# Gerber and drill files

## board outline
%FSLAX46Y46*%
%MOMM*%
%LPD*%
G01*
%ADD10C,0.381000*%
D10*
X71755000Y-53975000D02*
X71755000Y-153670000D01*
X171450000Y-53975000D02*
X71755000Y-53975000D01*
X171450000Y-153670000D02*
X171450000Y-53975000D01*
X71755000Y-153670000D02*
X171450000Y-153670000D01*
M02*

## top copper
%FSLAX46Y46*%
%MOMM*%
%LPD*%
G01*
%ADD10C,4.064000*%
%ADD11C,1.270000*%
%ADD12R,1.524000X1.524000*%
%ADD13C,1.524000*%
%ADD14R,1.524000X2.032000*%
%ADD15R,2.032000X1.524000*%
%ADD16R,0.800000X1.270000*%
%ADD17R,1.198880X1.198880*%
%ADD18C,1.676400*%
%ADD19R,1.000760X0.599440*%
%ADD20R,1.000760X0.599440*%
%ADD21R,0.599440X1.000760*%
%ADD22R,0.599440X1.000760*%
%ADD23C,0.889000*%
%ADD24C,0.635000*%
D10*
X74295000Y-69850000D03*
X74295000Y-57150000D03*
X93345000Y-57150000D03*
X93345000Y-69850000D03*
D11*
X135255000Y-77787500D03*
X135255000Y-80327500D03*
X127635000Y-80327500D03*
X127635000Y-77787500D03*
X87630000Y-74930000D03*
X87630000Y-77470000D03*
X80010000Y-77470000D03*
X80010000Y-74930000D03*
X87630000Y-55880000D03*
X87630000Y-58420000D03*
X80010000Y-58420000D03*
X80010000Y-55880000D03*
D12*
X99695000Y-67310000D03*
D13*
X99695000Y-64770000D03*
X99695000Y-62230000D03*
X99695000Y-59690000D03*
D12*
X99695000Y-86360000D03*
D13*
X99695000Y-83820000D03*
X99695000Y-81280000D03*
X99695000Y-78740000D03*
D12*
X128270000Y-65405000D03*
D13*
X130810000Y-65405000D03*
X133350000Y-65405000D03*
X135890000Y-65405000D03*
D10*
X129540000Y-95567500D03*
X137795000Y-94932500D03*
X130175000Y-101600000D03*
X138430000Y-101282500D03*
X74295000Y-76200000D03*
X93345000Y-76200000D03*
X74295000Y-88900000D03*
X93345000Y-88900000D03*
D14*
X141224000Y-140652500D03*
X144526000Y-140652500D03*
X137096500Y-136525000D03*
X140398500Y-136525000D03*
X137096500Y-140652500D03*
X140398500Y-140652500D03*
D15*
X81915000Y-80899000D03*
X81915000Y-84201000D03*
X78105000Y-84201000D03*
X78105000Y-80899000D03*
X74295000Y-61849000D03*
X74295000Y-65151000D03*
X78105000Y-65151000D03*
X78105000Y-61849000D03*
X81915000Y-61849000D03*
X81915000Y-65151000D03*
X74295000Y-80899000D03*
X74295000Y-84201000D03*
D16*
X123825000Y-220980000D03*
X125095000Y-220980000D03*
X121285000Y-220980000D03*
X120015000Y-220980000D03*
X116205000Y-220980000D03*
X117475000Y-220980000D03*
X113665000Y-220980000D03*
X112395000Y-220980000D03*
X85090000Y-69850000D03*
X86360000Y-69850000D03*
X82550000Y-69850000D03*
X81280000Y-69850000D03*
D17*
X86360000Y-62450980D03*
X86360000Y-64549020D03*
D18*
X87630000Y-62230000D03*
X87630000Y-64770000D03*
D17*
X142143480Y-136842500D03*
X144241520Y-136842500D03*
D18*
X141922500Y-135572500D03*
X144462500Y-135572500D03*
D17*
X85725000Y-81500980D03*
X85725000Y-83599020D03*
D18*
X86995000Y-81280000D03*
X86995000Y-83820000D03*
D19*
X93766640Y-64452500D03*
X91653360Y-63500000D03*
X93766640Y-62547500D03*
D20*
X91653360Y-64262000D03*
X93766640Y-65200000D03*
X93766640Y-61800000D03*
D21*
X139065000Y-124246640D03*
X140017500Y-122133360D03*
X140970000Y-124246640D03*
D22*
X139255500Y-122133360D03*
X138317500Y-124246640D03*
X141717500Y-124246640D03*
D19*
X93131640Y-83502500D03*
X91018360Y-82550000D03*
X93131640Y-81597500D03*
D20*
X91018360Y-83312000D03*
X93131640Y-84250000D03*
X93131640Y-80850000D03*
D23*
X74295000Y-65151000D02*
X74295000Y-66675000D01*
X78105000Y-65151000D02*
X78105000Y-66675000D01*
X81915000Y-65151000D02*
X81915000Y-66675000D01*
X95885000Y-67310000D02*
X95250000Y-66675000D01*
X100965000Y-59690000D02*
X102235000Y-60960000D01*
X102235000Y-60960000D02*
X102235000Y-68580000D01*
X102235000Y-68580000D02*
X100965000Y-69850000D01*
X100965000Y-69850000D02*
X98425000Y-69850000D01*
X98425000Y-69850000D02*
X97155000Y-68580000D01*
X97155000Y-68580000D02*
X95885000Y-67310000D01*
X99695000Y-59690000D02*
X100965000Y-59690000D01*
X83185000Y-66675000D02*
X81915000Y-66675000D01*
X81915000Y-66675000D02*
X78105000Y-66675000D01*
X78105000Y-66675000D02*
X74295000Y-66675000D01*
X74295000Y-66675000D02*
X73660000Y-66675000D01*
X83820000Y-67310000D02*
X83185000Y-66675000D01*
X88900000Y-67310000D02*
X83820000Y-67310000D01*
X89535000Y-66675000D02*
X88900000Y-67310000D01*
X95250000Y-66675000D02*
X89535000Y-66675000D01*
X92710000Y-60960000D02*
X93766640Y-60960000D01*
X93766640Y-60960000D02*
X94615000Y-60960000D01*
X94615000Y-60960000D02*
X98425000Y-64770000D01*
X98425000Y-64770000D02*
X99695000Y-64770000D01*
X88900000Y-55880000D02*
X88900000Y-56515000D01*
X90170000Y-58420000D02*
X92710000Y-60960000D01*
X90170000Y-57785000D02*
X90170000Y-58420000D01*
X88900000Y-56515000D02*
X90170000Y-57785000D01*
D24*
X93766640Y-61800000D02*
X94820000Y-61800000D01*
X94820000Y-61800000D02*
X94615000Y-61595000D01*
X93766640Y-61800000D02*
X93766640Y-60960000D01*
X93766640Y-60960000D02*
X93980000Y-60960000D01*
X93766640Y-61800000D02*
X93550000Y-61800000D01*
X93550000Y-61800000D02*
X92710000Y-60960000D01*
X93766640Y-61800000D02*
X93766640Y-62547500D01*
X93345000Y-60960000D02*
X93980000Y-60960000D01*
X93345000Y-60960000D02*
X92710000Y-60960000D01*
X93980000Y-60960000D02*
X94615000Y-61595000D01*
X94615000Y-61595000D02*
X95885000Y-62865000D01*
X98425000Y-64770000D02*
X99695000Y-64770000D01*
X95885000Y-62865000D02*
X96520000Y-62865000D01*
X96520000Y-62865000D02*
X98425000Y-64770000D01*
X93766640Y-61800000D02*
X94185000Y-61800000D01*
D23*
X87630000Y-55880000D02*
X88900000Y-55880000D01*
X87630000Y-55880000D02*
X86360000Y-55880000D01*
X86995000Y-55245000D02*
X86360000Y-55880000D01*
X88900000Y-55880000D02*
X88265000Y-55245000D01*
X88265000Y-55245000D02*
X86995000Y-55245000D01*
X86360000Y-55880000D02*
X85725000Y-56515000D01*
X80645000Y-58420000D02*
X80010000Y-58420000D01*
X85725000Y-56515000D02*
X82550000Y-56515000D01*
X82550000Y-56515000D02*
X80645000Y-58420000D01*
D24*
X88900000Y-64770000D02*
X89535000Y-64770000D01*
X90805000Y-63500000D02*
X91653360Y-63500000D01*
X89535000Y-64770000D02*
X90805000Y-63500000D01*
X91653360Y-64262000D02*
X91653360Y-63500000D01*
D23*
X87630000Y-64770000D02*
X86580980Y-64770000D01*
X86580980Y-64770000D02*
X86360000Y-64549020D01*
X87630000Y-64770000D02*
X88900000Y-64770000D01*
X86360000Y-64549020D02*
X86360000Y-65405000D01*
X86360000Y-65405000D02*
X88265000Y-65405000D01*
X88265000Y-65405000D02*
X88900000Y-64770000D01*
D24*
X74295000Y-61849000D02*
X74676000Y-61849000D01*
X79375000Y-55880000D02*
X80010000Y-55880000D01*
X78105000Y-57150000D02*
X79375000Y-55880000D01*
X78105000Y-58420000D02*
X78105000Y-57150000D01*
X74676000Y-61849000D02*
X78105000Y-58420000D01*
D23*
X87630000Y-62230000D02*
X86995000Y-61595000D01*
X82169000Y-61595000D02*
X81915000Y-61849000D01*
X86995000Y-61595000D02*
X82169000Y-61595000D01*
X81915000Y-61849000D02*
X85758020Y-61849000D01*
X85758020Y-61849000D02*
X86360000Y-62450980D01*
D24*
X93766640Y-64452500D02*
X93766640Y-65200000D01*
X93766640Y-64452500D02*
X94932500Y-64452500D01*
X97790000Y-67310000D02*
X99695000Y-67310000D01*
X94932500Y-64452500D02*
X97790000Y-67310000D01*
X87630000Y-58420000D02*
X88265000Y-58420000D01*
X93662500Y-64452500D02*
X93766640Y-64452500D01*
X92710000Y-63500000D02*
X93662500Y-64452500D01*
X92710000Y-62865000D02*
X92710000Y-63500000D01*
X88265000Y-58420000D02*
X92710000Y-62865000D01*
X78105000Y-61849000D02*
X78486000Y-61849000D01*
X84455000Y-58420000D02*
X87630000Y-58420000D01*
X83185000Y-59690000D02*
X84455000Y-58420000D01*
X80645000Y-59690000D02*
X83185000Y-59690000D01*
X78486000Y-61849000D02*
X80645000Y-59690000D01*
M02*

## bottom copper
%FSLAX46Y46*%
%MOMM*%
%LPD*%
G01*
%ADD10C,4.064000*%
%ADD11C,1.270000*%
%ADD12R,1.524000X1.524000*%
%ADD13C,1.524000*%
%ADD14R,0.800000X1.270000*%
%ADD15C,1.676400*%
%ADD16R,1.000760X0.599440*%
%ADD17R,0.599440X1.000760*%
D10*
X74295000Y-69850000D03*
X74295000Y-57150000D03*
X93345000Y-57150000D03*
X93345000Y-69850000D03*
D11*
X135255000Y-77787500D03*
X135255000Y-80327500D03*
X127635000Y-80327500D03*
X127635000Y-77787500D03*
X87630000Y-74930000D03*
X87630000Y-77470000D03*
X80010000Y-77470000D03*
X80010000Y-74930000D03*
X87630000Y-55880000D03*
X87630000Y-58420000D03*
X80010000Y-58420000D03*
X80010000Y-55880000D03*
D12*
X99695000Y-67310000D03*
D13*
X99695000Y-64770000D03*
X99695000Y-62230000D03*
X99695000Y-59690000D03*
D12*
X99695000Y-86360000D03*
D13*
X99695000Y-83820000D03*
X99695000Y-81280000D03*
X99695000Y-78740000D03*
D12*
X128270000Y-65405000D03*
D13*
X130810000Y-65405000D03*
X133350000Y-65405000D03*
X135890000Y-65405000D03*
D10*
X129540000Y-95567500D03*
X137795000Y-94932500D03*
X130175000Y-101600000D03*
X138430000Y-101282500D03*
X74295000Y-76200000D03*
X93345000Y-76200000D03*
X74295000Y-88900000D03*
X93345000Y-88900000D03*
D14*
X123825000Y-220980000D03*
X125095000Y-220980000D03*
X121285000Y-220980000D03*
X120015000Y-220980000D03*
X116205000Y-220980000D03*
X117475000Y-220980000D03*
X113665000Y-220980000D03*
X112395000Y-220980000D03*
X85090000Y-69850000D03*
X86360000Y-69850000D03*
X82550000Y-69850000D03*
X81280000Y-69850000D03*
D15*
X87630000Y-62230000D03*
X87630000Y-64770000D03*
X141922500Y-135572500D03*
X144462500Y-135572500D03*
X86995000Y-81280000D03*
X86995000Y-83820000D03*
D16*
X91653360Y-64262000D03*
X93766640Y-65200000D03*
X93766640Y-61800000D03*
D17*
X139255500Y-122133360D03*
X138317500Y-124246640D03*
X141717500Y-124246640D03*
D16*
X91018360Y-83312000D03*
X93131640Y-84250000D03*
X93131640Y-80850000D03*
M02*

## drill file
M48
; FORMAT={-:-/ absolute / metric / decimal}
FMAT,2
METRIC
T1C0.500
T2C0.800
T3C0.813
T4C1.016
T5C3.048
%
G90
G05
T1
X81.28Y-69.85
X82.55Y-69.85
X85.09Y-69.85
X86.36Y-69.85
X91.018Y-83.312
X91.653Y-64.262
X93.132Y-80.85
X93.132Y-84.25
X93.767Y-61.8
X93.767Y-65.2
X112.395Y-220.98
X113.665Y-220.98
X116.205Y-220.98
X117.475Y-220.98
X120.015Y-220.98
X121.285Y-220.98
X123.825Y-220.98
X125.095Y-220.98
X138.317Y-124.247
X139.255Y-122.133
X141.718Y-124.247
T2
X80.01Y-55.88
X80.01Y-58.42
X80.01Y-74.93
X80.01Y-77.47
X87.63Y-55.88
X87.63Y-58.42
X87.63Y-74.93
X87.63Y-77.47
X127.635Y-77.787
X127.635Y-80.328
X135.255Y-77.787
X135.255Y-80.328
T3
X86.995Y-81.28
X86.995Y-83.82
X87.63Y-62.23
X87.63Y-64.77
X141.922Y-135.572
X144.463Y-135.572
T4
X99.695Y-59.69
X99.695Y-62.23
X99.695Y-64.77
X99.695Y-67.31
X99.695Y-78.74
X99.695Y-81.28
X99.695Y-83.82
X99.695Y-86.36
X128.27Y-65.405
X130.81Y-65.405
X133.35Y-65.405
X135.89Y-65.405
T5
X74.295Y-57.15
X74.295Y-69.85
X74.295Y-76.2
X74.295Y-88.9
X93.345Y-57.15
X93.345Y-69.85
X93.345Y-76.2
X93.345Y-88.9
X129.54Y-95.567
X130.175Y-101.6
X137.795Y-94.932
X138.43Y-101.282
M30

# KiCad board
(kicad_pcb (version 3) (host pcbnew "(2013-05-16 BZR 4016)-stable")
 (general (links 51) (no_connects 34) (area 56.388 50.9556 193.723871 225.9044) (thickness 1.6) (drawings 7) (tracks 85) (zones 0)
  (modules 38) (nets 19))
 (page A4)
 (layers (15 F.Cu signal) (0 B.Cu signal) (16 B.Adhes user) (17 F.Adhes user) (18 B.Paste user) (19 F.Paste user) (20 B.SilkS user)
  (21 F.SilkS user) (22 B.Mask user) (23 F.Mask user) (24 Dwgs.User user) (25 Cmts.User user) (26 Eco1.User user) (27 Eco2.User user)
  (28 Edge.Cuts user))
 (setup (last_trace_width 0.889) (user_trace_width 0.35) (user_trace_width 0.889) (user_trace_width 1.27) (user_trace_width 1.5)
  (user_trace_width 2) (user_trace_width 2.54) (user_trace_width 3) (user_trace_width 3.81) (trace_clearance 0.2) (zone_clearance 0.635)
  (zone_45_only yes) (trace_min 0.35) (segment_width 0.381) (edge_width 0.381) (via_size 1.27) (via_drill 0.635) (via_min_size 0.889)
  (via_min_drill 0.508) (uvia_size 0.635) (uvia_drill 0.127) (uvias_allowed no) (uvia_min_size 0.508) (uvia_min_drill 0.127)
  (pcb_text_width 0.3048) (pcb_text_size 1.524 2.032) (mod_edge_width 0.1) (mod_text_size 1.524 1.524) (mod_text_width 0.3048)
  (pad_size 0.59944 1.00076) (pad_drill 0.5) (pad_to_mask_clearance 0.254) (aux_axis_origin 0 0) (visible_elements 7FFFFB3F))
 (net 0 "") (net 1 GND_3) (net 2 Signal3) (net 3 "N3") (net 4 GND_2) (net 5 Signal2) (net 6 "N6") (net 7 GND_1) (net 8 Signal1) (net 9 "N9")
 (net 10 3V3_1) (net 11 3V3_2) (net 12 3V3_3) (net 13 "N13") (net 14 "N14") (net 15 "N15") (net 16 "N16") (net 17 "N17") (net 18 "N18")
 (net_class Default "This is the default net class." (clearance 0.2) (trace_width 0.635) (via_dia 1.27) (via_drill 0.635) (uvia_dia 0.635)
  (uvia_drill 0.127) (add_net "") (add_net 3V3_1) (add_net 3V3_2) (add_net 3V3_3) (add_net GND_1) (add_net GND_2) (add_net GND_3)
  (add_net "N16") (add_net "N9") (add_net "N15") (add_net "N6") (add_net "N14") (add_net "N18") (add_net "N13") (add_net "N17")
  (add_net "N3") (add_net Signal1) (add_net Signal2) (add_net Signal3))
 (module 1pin (layer F.Cu) (at 74.295 69.85)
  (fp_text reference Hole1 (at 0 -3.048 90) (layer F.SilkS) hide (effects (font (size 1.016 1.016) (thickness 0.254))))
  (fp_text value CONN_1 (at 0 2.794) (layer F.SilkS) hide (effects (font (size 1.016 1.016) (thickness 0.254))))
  (pad 1 thru_hole circle (at 0 0) (size 4.064 4.064) (drill 3.048) (layers *.Cu *.Mask F.SilkS)))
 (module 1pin (layer F.Cu) (at 74.295 57.15)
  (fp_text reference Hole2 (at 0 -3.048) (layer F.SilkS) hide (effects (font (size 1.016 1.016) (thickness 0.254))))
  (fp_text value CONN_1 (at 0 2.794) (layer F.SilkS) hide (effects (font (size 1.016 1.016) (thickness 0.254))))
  (pad 1 thru_hole circle (at 0 0) (size 4.064 4.064) (drill 3.048) (layers *.Cu *.Mask F.SilkS)))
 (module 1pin (layer F.Cu) (at 93.345 57.15)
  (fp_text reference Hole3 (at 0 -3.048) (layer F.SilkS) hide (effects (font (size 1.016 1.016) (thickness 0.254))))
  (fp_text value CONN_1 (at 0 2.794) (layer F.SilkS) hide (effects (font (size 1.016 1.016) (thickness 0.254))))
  (pad 1 thru_hole circle (at 0 0) (size 4.064 4.064) (drill 3.048) (layers *.Cu *.Mask F.SilkS)))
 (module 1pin (layer F.Cu) (at 93.345 69.85)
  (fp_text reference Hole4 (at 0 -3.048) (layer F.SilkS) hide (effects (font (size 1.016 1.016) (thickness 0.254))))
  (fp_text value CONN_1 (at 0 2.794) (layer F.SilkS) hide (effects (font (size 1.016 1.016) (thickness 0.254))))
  (pad 1 thru_hole circle (at 0 0) (size 4.064 4.064) (drill 3.048) (layers *.Cu *.Mask F.SilkS)))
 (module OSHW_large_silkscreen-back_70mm (layer B.Cu) (at 146.685 185.42)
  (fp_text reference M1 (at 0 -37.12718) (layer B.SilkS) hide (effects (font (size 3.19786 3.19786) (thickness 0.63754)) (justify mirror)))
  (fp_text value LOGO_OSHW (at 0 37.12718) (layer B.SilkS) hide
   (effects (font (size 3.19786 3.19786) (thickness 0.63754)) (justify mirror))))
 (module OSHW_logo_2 (layer F.Cu) (at 187.96 158.75)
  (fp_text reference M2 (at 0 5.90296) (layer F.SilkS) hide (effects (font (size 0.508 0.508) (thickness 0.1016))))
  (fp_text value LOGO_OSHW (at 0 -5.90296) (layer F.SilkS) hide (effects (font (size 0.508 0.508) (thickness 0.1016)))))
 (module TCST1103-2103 (layer F.Cu) (at 131.445 79.0575)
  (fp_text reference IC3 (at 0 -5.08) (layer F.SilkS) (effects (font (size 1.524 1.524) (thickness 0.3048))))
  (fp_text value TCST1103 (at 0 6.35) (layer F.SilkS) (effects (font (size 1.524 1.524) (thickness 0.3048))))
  (pad E/D thru_hole circle (at 3.81 -1.27) (size 1.27 1.27) (drill 0.8) (layers *.Cu *.Mask F.SilkS) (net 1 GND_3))
  (pad C/+ thru_hole circle (at 3.81 1.27) (size 1.27 1.27) (drill 0.8) (layers *.Cu *.Mask F.SilkS) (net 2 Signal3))
  (pad K/E thru_hole circle (at -3.81 1.27) (size 1.27 1.27) (drill 0.8) (layers *.Cu *.Mask F.SilkS) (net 1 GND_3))
  (pad A/+ thru_hole circle (at -3.81 -1.27) (size 1.27 1.27) (drill 0.8) (layers *.Cu *.Mask F.SilkS) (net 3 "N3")))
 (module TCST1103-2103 (layer F.Cu) (at 83.82 76.2)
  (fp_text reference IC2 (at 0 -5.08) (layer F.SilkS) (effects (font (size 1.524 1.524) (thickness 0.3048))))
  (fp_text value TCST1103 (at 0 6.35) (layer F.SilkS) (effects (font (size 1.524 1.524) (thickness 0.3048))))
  (pad E/D thru_hole circle (at 3.81 -1.27) (size 1.27 1.27) (drill 0.8) (layers *.Cu *.Mask F.SilkS) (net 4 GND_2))
  (pad C/+ thru_hole circle (at 3.81 1.27) (size 1.27 1.27) (drill 0.8) (layers *.Cu *.Mask F.SilkS) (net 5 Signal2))
  (pad K/E thru_hole circle (at -3.81 1.27) (size 1.27 1.27) (drill 0.8) (layers *.Cu *.Mask F.SilkS) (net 4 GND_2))
  (pad A/+ thru_hole circle (at -3.81 -1.27) (size 1.27 1.27) (drill 0.8) (layers *.Cu *.Mask F.SilkS) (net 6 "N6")))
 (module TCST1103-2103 (layer F.Cu) (at 83.82 57.15)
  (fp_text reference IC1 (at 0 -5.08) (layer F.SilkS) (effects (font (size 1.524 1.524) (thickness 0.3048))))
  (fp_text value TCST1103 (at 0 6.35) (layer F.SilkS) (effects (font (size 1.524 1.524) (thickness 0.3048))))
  (pad E/D thru_hole circle (at 3.81 -1.27) (size 1.27 1.27) (drill 0.8) (layers *.Cu *.Mask F.SilkS) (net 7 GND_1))
  (pad C/+ thru_hole circle (at 3.81 1.27) (size 1.27 1.27) (drill 0.8) (layers *.Cu *.Mask F.SilkS) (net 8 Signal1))
  (pad K/E thru_hole circle (at -3.81 1.27) (size 1.27 1.27) (drill 0.8) (layers *.Cu *.Mask F.SilkS) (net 7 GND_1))
  (pad A/+ thru_hole circle (at -3.81 -1.27) (size 1.27 1.27) (drill 0.8) (layers *.Cu *.Mask F.SilkS) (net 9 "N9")))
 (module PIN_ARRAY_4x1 (layer F.Cu) (at 99.695 63.5 90)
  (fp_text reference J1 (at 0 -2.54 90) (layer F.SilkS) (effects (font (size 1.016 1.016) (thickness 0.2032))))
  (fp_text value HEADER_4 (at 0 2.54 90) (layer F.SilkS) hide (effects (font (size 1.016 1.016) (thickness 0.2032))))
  (pad 1 thru_hole rect (at -3.81 0 90) (size 1.524 1.524) (drill 1.016) (layers *.Cu *.Mask F.SilkS) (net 8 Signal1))
  (pad 2 thru_hole circle (at -1.27 0 90) (size 1.524 1.524) (drill 1.016) (layers *.Cu *.Mask F.SilkS) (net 7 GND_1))
  (pad 3 thru_hole circle (at 1.27 0 90) (size 1.524 1.524) (drill 1.016) (layers *.Cu *.Mask F.SilkS))
  (pad 4 thru_hole circle (at 3.81 0 90) (size 1.524 1.524) (drill 1.016) (layers *.Cu *.Mask F.SilkS) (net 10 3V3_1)))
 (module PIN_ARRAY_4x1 (layer F.Cu) (at 99.695 82.55 90)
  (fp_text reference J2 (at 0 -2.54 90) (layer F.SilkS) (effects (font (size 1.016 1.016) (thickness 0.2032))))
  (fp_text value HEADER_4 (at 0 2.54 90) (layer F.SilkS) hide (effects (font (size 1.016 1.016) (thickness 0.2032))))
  (pad 1 thru_hole rect (at -3.81 0 90) (size 1.524 1.524) (drill 1.016) (layers *.Cu *.Mask F.SilkS) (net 5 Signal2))
  (pad 2 thru_hole circle (at -1.27 0 90) (size 1.524 1.524) (drill 1.016) (layers *.Cu *.Mask F.SilkS) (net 4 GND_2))
  (pad 3 thru_hole circle (at 1.27 0 90) (size 1.524 1.524) (drill 1.016) (layers *.Cu *.Mask F.SilkS))
  (pad 4 thru_hole circle (at 3.81 0 90) (size 1.524 1.524) (drill 1.016) (layers *.Cu *.Mask F.SilkS) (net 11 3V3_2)))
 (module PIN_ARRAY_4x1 (layer F.Cu) (at 132.08 65.405)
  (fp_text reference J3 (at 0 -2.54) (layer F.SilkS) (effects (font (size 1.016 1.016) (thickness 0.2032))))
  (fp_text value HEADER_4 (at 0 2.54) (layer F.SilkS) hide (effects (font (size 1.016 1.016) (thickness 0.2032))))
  (pad 1 thru_hole rect (at -3.81 0) (size 1.524 1.524) (drill 1.016) (layers *.Cu *.Mask F.SilkS) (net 2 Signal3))
  (pad 2 thru_hole circle (at -1.27 0) (size 1.524 1.524) (drill 1.016) (layers *.Cu *.Mask F.SilkS) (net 1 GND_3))
  (pad 3 thru_hole circle (at 1.27 0) (size 1.524 1.524) (drill 1.016) (layers *.Cu *.Mask F.SilkS))
  (pad 4 thru_hole circle (at 3.81 0) (size 1.524 1.524) (drill 1.016) (layers *.Cu *.Mask F.SilkS) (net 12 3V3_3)))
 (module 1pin (layer F.Cu) (at 129.54 95.5675)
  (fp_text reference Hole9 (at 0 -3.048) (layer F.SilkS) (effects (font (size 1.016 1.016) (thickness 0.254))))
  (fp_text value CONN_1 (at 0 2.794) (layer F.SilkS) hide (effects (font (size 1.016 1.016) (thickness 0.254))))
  (pad 1 thru_hole circle (at 0 0) (size 4.064 4.064) (drill 3.048) (layers *.Cu *.Mask F.SilkS)))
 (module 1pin (layer F.Cu) (at 137.795 94.9325)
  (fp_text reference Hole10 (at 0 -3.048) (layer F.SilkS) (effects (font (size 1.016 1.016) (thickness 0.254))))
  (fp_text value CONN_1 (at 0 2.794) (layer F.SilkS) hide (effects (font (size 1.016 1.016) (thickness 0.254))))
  (pad 1 thru_hole circle (at 0 0) (size 4.064 4.064) (drill 3.048) (layers *.Cu *.Mask F.SilkS)))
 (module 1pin (layer F.Cu) (at 130.175 101.6)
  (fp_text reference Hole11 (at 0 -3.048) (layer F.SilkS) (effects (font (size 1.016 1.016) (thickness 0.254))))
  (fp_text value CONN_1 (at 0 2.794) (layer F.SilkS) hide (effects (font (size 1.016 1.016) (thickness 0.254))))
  (pad 1 thru_hole circle (at 0 0) (size 4.064 4.064) (drill 3.048) (layers *.Cu *.Mask F.SilkS)))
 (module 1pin (layer F.Cu) (at 138.43 101.2825)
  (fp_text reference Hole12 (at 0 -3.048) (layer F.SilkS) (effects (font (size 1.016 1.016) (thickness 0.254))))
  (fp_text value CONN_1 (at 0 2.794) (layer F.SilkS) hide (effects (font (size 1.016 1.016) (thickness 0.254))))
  (pad 1 thru_hole circle (at 0 0) (size 4.064 4.064) (drill 3.048) (layers *.Cu *.Mask F.SilkS)))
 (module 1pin (layer F.Cu) (at 74.295 76.2)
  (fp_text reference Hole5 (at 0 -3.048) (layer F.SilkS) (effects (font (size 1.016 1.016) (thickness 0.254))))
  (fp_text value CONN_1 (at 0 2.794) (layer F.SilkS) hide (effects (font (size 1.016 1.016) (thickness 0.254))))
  (pad 1 thru_hole circle (at 0 0) (size 4.064 4.064) (drill 3.048) (layers *.Cu *.Mask F.SilkS)))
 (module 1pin (layer F.Cu) (at 93.345 76.2)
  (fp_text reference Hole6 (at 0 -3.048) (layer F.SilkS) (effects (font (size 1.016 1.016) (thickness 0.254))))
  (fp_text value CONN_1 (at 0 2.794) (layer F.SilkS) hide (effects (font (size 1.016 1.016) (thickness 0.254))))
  (pad 1 thru_hole circle (at 0 0) (size 4.064 4.064) (drill 3.048) (layers *.Cu *.Mask F.SilkS)))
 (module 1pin (layer F.Cu) (at 74.295 88.9)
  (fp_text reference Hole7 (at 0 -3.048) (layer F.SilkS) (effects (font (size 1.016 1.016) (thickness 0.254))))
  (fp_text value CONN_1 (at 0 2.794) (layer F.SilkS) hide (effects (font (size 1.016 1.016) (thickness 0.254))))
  (pad 1 thru_hole circle (at 0 0) (size 4.064 4.064) (drill 3.048) (layers *.Cu *.Mask F.SilkS)))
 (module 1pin (layer F.Cu) (at 93.345 88.9)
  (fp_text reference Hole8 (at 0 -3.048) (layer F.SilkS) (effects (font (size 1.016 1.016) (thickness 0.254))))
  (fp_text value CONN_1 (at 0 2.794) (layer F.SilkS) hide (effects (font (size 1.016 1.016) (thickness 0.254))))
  (pad 1 thru_hole circle (at 0 0) (size 4.064 4.064) (drill 3.048) (layers *.Cu *.Mask F.SilkS)))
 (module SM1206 (layer F.Cu) (at 142.875 140.6525)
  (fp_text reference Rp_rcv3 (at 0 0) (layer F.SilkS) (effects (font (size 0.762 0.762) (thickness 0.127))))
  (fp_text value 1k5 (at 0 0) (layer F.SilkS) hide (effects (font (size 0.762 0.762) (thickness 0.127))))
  (pad 1 smd rect (at -1.651 0) (size 1.524 2.032) (layers F.Cu F.Paste F.Mask) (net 12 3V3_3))
  (pad 2 smd rect (at 1.651 0) (size 1.524 2.032) (layers F.Cu F.Paste F.Mask) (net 2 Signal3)))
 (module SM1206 (layer F.Cu) (at 138.7475 136.525)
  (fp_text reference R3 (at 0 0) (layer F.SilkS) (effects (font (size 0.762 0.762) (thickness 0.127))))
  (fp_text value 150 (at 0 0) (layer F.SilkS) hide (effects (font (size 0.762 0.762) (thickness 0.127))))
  (pad 1 smd rect (at -1.651 0) (size 1.524 2.032) (layers F.Cu F.Paste F.Mask) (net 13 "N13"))
  (pad 2 smd rect (at 1.651 0) (size 1.524 2.032) (layers F.Cu F.Paste F.Mask) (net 12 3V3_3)))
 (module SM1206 (layer F.Cu) (at 138.7475 140.6525)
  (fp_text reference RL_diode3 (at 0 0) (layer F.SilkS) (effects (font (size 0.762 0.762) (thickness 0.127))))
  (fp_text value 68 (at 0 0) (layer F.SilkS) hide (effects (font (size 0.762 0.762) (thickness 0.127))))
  (pad 1 smd rect (at -1.651 0) (size 1.524 2.032) (layers F.Cu F.Paste F.Mask) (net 3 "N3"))
  (pad 2 smd rect (at 1.651 0) (size 1.524 2.032) (layers F.Cu F.Paste F.Mask) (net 12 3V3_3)))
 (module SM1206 (layer F.Cu) (at 81.915 82.55 270)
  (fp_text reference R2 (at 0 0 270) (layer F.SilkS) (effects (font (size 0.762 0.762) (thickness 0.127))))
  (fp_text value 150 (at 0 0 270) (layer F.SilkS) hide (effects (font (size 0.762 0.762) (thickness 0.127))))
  (pad 1 smd rect (at -1.651 0 270) (size 1.524 2.032) (layers F.Cu F.Paste F.Mask) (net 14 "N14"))
  (pad 2 smd rect (at 1.651 0 270) (size 1.524 2.032) (layers F.Cu F.Paste F.Mask) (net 11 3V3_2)))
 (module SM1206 (layer F.Cu) (at 78.105 82.55 90)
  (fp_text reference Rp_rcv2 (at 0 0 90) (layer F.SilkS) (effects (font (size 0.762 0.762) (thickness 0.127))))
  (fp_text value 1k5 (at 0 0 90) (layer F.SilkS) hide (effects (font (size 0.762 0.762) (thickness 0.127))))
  (pad 1 smd rect (at -1.651 0 90) (size 1.524 2.032) (layers F.Cu F.Paste F.Mask) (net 11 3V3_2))
  (pad 2 smd rect (at 1.651 0 90) (size 1.524 2.032) (layers F.Cu F.Paste F.Mask) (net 5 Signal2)))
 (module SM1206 (layer F.Cu) (at 74.295 63.5 270)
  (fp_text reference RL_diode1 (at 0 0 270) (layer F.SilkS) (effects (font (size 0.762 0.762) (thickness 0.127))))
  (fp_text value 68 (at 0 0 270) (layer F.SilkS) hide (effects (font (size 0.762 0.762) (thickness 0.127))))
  (pad 1 smd rect (at -1.651 0 270) (size 1.524 2.032) (layers F.Cu F.Paste F.Mask) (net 9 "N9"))
  (pad 2 smd rect (at 1.651 0 270) (size 1.524 2.032) (layers F.Cu F.Paste F.Mask) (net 10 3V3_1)))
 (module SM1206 (layer F.Cu) (at 78.105 63.5 90)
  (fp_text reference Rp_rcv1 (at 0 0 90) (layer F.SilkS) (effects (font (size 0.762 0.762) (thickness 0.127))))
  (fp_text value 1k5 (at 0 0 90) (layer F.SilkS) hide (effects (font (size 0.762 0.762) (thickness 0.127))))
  (pad 1 smd rect (at -1.651 0 90) (size 1.524 2.032) (layers F.Cu F.Paste F.Mask) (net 10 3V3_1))
  (pad 2 smd rect (at 1.651 0 90) (size 1.524 2.032) (layers F.Cu F.Paste F.Mask) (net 8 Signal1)))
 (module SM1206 (layer F.Cu) (at 81.915 63.5 270)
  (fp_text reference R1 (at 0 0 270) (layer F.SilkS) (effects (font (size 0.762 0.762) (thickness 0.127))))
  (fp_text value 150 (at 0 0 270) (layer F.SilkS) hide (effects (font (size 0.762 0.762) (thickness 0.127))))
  (pad 1 smd rect (at -1.651 0 270) (size 1.524 2.032) (layers F.Cu F.Paste F.Mask) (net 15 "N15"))
  (pad 2 smd rect (at 1.651 0 270) (size 1.524 2.032) (layers F.Cu F.Paste F.Mask) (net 10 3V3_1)))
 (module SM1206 (layer F.Cu) (at 74.295 82.55 270)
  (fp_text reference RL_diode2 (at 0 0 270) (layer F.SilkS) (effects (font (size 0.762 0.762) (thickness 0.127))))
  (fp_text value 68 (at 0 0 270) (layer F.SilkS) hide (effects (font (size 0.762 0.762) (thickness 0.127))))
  (pad 1 smd rect (at -1.651 0 270) (size 1.524 2.032) (layers F.Cu F.Paste F.Mask) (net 6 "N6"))
  (pad 2 smd rect (at 1.651 0 270) (size 1.524 2.032) (layers F.Cu F.Paste F.Mask) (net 11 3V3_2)))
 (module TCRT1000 (layer F.Cu) (at 122.555 220.98)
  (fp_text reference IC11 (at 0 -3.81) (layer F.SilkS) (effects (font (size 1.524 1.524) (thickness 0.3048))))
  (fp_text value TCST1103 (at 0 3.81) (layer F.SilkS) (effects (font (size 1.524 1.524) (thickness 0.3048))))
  (pad E/D thru_hole rect (at 1.27 0) (size 0.8 1.27) (drill 0.5) (layers *.Cu *.Mask F.SilkS))
  (pad C/+ thru_hole rect (at 2.54 0) (size 0.8 1.27) (drill 0.5) (layers *.Cu *.Mask F.SilkS))
  (pad K/E thru_hole rect (at -1.27 0) (size 0.8 1.27) (drill 0.5) (layers *.Cu *.Mask F.SilkS))
  (pad A/+ thru_hole rect (at -2.54 0) (size 0.8 1.27) (drill 0.5) (layers *.Cu *.Mask F.SilkS)))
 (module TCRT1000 (layer F.Cu) (at 114.935 220.98)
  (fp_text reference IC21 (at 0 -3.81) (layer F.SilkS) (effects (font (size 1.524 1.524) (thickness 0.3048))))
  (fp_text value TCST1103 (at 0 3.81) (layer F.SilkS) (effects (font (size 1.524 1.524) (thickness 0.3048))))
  (pad E/D thru_hole rect (at 1.27 0) (size 0.8 1.27) (drill 0.5) (layers *.Cu *.Mask F.SilkS))
  (pad C/+ thru_hole rect (at 2.54 0) (size 0.8 1.27) (drill 0.5) (layers *.Cu *.Mask F.SilkS))
  (pad K/E thru_hole rect (at -1.27 0) (size 0.8 1.27) (drill 0.5) (layers *.Cu *.Mask F.SilkS))
  (pad A/+ thru_hole rect (at -2.54 0) (size 0.8 1.27) (drill 0.5) (layers *.Cu *.Mask F.SilkS)))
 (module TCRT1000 (layer F.Cu) (at 83.82 69.85)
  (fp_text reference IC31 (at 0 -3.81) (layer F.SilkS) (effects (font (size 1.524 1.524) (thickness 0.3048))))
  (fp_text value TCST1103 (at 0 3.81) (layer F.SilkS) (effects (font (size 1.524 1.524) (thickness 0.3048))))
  (pad E/D thru_hole rect (at 1.27 0) (size 0.8 1.27) (drill 0.5) (layers *.Cu *.Mask F.SilkS))
  (pad C/+ thru_hole rect (at 2.54 0) (size 0.8 1.27) (drill 0.5) (layers *.Cu *.Mask F.SilkS))
  (pad K/E thru_hole rect (at -1.27 0) (size 0.8 1.27) (drill 0.5) (layers *.Cu *.Mask F.SilkS))
  (pad A/+ thru_hole rect (at -2.54 0) (size 0.8 1.27) (drill 0.5) (layers *.Cu *.Mask F.SilkS)))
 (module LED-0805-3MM (layer F.Cu) (at 86.36 63.5 270)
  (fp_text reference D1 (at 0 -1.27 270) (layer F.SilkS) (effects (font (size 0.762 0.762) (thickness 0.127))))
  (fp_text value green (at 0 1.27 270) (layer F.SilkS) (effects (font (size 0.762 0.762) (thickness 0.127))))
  (pad 1 smd rect (at -1.04902 0 270) (size 1.19888 1.19888) (layers F.Cu F.Paste F.Mask) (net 15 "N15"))
  (pad 2 smd rect (at 1.04902 0 270) (size 1.19888 1.19888) (layers F.Cu F.Paste F.Mask) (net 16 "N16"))
  (pad 1 thru_hole circle (at -1.27 -1.27 270) (size 1.6764 1.6764) (drill 0.8128) (layers *.Cu *.Mask F.SilkS) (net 15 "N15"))
  (pad 2 thru_hole circle (at 1.27 -1.27 270) (size 1.6764 1.6764) (drill 0.8128) (layers *.Cu *.Mask F.SilkS) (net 16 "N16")))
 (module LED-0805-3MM (layer F.Cu) (at 143.1925 136.8425)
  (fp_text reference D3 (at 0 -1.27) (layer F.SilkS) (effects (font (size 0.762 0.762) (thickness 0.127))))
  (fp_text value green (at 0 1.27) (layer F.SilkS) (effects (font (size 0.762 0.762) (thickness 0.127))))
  (pad 1 smd rect (at -1.04902 0) (size 1.19888 1.19888) (layers F.Cu F.Paste F.Mask) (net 13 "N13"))
  (pad 2 smd rect (at 1.04902 0) (size 1.19888 1.19888) (layers F.Cu F.Paste F.Mask) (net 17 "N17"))
  (pad 1 thru_hole circle (at -1.27 -1.27) (size 1.6764 1.6764) (drill 0.8128) (layers *.Cu *.Mask F.SilkS) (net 13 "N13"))
  (pad 2 thru_hole circle (at 1.27 -1.27) (size 1.6764 1.6764) (drill 0.8128) (layers *.Cu *.Mask F.SilkS) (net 17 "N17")))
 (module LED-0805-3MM (layer F.Cu) (at 85.725 82.55 270)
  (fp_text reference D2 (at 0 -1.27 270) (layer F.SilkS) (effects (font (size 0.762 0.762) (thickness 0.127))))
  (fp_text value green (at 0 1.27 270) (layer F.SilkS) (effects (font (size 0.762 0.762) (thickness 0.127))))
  (pad 1 smd rect (at -1.04902 0 270) (size 1.19888 1.19888) (layers F.Cu F.Paste F.Mask) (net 14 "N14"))
  (pad 2 smd rect (at 1.04902 0 270) (size 1.19888 1.19888) (layers F.Cu F.Paste F.Mask) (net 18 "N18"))
  (pad 1 thru_hole circle (at -1.27 -1.27 270) (size 1.6764 1.6764) (drill 0.8128) (layers *.Cu *.Mask F.SilkS) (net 14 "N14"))
  (pad 2 thru_hole circle (at 1.27 -1.27 270) (size 1.6764 1.6764) (drill 0.8128) (layers *.Cu *.Mask F.SilkS) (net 18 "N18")))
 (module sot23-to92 (layer F.Cu) (at 92.71 63.5 90)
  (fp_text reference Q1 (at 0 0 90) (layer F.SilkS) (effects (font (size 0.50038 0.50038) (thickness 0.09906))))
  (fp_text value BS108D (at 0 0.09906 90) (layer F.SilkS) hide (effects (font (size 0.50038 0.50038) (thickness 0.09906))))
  (pad G smd rect (at -0.9525 1.05664 90) (size 0.59944 1.00076) (layers F.Cu F.Paste F.Mask) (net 8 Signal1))
  (pad D smd rect (at 0 -1.05664 90) (size 0.59944 1.00076) (layers F.Cu F.Paste F.Mask) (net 16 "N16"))
  (pad S smd rect (at 0.9525 1.05664 90) (size 0.59944 1.00076) (layers F.Cu F.Paste F.Mask) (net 7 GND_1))
  (pad D thru_hole rect (at -0.762 -1.05664 90) (size 0.59944 1.00076) (drill 0.5) (layers *.Cu *.Mask F.SilkS) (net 16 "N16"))
  (pad G thru_hole rect (at -1.7 1.05664 90) (size 0.59944 1.00076) (drill 0.5) (layers *.Cu *.Mask F.SilkS) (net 8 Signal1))
  (pad S thru_hole rect (at 1.7 1.05664 90) (size 0.59944 1.00076) (drill 0.5) (layers *.Cu *.Mask F.SilkS) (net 7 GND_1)))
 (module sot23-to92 (layer F.Cu) (at 140.0175 123.19)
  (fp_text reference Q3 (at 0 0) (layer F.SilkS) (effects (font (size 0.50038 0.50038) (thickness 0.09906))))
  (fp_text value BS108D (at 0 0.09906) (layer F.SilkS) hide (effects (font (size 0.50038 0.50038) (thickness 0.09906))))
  (pad G smd rect (at -0.9525 1.05664) (size 0.59944 1.00076) (layers F.Cu F.Paste F.Mask) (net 2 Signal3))
  (pad D smd rect (at 0 -1.05664) (size 0.59944 1.00076) (layers F.Cu F.Paste F.Mask) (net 17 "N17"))
  (pad S smd rect (at 0.9525 1.05664) (size 0.59944 1.00076) (layers F.Cu F.Paste F.Mask) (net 1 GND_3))
  (pad D thru_hole rect (at -0.762 -1.05664) (size 0.59944 1.00076) (drill 0.5) (layers *.Cu *.Mask F.SilkS) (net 17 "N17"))
  (pad G thru_hole rect (at -1.7 1.05664) (size 0.59944 1.00076) (drill 0.5) (layers *.Cu *.Mask F.SilkS) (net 2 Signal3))
  (pad S thru_hole rect (at 1.7 1.05664) (size 0.59944 1.00076) (drill 0.5) (layers *.Cu *.Mask F.SilkS) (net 1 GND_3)))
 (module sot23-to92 (layer F.Cu) (at 92.075 82.55 90)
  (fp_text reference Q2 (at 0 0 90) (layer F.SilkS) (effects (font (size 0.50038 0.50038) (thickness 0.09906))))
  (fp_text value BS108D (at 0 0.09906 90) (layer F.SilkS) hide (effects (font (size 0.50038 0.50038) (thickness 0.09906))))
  (pad G smd rect (at -0.9525 1.05664 90) (size 0.59944 1.00076) (layers F.Cu F.Paste F.Mask) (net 5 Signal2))
  (pad D smd rect (at 0 -1.05664 90) (size 0.59944 1.00076) (layers F.Cu F.Paste F.Mask) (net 18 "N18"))
  (pad S smd rect (at 0.9525 1.05664 90) (size 0.59944 1.00076) (layers F.Cu F.Paste F.Mask) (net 4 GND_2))
  (pad D thru_hole rect (at -0.762 -1.05664 90) (size 0.59944 1.00076) (drill 0.5) (layers *.Cu *.Mask F.SilkS) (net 18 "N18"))
  (pad G thru_hole rect (at -1.7 1.05664 90) (size 0.59944 1.00076) (drill 0.5) (layers *.Cu *.Mask F.SilkS) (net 5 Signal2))
  (pad S thru_hole rect (at 1.7 1.05664 90) (size 0.59944 1.00076) (drill 0.5) (layers *.Cu *.Mask F.SilkS) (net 4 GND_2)))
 (gr_line (start 71.755 53.975) (end 71.755 153.67) (angle 90) (layer Edge.Cuts) (width 0.381))
 (gr_line (start 171.45 53.975) (end 71.755 53.975) (angle 90) (layer Edge.Cuts) (width 0.381))
 (gr_line (start 171.45 153.67) (end 171.45 53.975) (angle 90) (layer Edge.Cuts) (width 0.381))
 (gr_line (start 71.755 153.67) (end 171.45 153.67) (angle 90) (layer Edge.Cuts) (width 0.381))
 (segment (start 74.295 65.151) (end 74.295 66.675) (width 0.889) (layer F.Cu) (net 10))
 (segment (start 78.105 65.151) (end 78.105 66.675) (width 0.889) (layer F.Cu) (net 10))
 (segment (start 81.915 65.151) (end 81.915 66.675) (width 0.889) (layer F.Cu) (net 10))
 (segment (start 95.885 67.31) (end 95.25 66.675) (width 0.889) (layer F.Cu) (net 10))
 (segment (start 100.965 59.69) (end 102.235 60.96) (width 0.889) (layer F.Cu) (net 10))
 (segment (start 102.235 60.96) (end 102.235 68.58) (width 0.889) (layer F.Cu) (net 10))
 (segment (start 102.235 68.58) (end 100.965 69.85) (width 0.889) (layer F.Cu) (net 10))
 (segment (start 100.965 69.85) (end 98.425 69.85) (width 0.889) (layer F.Cu) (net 10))
 (segment (start 98.425 69.85) (end 97.155 68.58) (width 0.889) (layer F.Cu) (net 10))
 (segment (start 97.155 68.58) (end 95.885 67.31) (width 0.889) (layer F.Cu) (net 10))
 (segment (start 99.695 59.69) (end 100.965 59.69) (width 0.889) (layer F.Cu) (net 10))
 (segment (start 83.185 66.675) (end 81.915 66.675) (width 0.889) (layer F.Cu) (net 10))
 (segment (start 81.915 66.675) (end 78.105 66.675) (width 0.889) (layer F.Cu) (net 10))
 (segment (start 78.105 66.675) (end 74.295 66.675) (width 0.889) (layer F.Cu) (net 10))
 (segment (start 74.295 66.675) (end 73.66 66.675) (width 0.889) (layer F.Cu) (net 10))
 (segment (start 83.82 67.31) (end 83.185 66.675) (width 0.889) (layer F.Cu) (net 10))
 (segment (start 88.9 67.31) (end 83.82 67.31) (width 0.889) (layer F.Cu) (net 10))
 (segment (start 89.535 66.675) (end 88.9 67.31) (width 0.889) (layer F.Cu) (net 10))
 (segment (start 95.25 66.675) (end 89.535 66.675) (width 0.889) (layer F.Cu) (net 10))
 (segment (start 92.71 60.96) (end 93.76664 60.96) (width 0.889) (layer F.Cu) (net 7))
 (segment (start 93.76664 60.96) (end 94.615 60.96) (width 0.889) (layer F.Cu) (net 7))
 (segment (start 94.615 60.96) (end 98.425 64.77) (width 0.889) (layer F.Cu) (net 7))
 (segment (start 98.425 64.77) (end 99.695 64.77) (width 0.889) (layer F.Cu) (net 7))
 (segment (start 88.9 55.88) (end 88.9 56.515) (width 0.889) (layer F.Cu) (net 7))
 (segment (start 90.17 58.42) (end 92.71 60.96) (width 0.889) (layer F.Cu) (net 7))
 (segment (start 90.17 57.785) (end 90.17 58.42) (width 0.889) (layer F.Cu) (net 7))
 (segment (start 88.9 56.515) (end 90.17 57.785) (width 0.889) (layer F.Cu) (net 7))
 (segment (start 93.76664 61.8) (end 94.82 61.8) (width 0.635) (layer F.Cu) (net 7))
 (segment (start 94.82 61.8) (end 94.615 61.595) (width 0.635) (layer F.Cu) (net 7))
 (segment (start 93.76664 61.8) (end 93.76664 60.96) (width 0.635) (layer F.Cu) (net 7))
 (segment (start 93.76664 60.96) (end 93.98 60.96) (width 0.635) (layer F.Cu) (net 7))
 (segment (start 93.76664 61.8) (end 93.55 61.8) (width 0.635) (layer F.Cu) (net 7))
 (segment (start 93.55 61.8) (end 92.71 60.96) (width 0.635) (layer F.Cu) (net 7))
 (segment (start 93.76664 61.8) (end 93.76664 62.5475) (width 0.635) (layer F.Cu) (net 7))
 (segment (start 93.345 60.96) (end 93.98 60.96) (width 0.635) (layer F.Cu) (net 7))
 (segment (start 93.345 60.96) (end 92.71 60.96) (width 0.635) (layer F.Cu) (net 7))
 (segment (start 93.98 60.96) (end 94.615 61.595) (width 0.635) (layer F.Cu) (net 7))
 (segment (start 94.615 61.595) (end 95.885 62.865) (width 0.635) (layer F.Cu) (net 7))
 (segment (start 98.425 64.77) (end 99.695 64.77) (width 0.635) (layer F.Cu) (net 7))
 (segment (start 95.885 62.865) (end 96.52 62.865) (width 0.635) (layer F.Cu) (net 7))
 (segment (start 96.52 62.865) (end 98.425 64.77) (width 0.635) (layer F.Cu) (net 7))
 (segment (start 93.76664 61.8) (end 94.185 61.8) (width 0.635) (layer F.Cu) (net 7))
 (segment (start 87.63 55.88) (end 88.9 55.88) (width 0.889) (layer F.Cu) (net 7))
 (segment (start 87.63 55.88) (end 86.36 55.88) (width 0.889) (layer F.Cu) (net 7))
 (segment (start 86.995 55.245) (end 86.36 55.88) (width 0.889) (layer F.Cu) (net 7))
 (segment (start 88.9 55.88) (end 88.265 55.245) (width 0.889) (layer F.Cu) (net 7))
 (segment (start 88.265 55.245) (end 86.995 55.245) (width 0.889) (layer F.Cu) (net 7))
 (segment (start 86.36 55.88) (end 85.725 56.515) (width 0.889) (layer F.Cu) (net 7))
 (segment (start 80.645 58.42) (end 80.01 58.42) (width 0.889) (layer F.Cu) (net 7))
 (segment (start 85.725 56.515) (end 82.55 56.515) (width 0.889) (layer F.Cu) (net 7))
 (segment (start 82.55 56.515) (end 80.645 58.42) (width 0.889) (layer F.Cu) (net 7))
 (segment (start 88.9 64.77) (end 89.535 64.77) (width 0.635) (layer F.Cu) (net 16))
 (segment (start 90.805 63.5) (end 91.65336 63.5) (width 0.635) (layer F.Cu) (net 16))
 (segment (start 89.535 64.77) (end 90.805 63.5) (width 0.635) (layer F.Cu) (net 16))
 (segment (start 91.65336 64.262) (end 91.65336 63.5) (width 0.635) (layer F.Cu) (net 16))
 (segment (start 87.63 64.77) (end 86.58098 64.77) (width 0.889) (layer F.Cu) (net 16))
 (segment (start 86.58098 64.77) (end 86.36 64.54902) (width 0.889) (layer F.Cu) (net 16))
 (segment (start 87.63 64.77) (end 88.9 64.77) (width 0.889) (layer F.Cu) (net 16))
 (segment (start 86.36 64.54902) (end 86.36 65.405) (width 0.889) (layer F.Cu) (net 16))
 (segment (start 86.36 65.405) (end 88.265 65.405) (width 0.889) (layer F.Cu) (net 16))
 (segment (start 88.265 65.405) (end 88.9 64.77) (width 0.889) (layer F.Cu) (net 16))
 (segment (start 74.295 61.849) (end 74.676 61.849) (width 0.635) (layer F.Cu) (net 9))
 (segment (start 79.375 55.88) (end 80.01 55.88) (width 0.635) (layer F.Cu) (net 9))
 (segment (start 78.105 57.15) (end 79.375 55.88) (width 0.635) (layer F.Cu) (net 9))
 (segment (start 78.105 58.42) (end 78.105 57.15) (width 0.635) (layer F.Cu) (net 9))
 (segment (start 74.676 61.849) (end 78.105 58.42) (width 0.635) (layer F.Cu) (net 9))
 (segment (start 87.63 62.23) (end 86.995 61.595) (width 0.889) (layer F.Cu) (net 15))
 (segment (start 82.169 61.595) (end 81.915 61.849) (width 0.889) (layer F.Cu) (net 15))
 (segment (start 86.995 61.595) (end 82.169 61.595) (width 0.889) (layer F.Cu) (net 15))
 (segment (start 81.915 61.849) (end 85.75802 61.849) (width 0.889) (layer F.Cu) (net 15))
 (segment (start 85.75802 61.849) (end 86.36 62.45098) (width 0.889) (layer F.Cu) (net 15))
 (segment (start 93.76664 64.4525) (end 93.76664 65.2) (width 0.635) (layer F.Cu) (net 8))
 (segment (start 93.76664 64.4525) (end 94.9325 64.4525) (width 0.635) (layer F.Cu) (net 8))
 (segment (start 97.79 67.31) (end 99.695 67.31) (width 0.635) (layer F.Cu) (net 8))
 (segment (start 94.9325 64.4525) (end 97.79 67.31) (width 0.635) (layer F.Cu) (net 8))
 (segment (start 87.63 58.42) (end 88.265 58.42) (width 0.635) (layer F.Cu) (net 8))
 (segment (start 93.6625 64.4525) (end 93.76664 64.4525) (width 0.635) (layer F.Cu) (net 8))
 (segment (start 92.71 63.5) (end 93.6625 64.4525) (width 0.635) (layer F.Cu) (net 8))
 (segment (start 92.71 62.865) (end 92.71 63.5) (width 0.635) (layer F.Cu) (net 8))
 (segment (start 88.265 58.42) (end 92.71 62.865) (width 0.635) (layer F.Cu) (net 8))
 (segment (start 78.105 61.849) (end 78.486 61.849) (width 0.635) (layer F.Cu) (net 8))
 (segment (start 84.455 58.42) (end 87.63 58.42) (width 0.635) (layer F.Cu) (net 8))
 (segment (start 83.185 59.69) (end 84.455 58.42) (width 0.635) (layer F.Cu) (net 8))
 (segment (start 80.645 59.69) (end 83.185 59.69) (width 0.635) (layer F.Cu) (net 8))
 (segment (start 78.486 61.849) (end 80.645 59.69) (width 0.635) (layer F.Cu) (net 8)))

